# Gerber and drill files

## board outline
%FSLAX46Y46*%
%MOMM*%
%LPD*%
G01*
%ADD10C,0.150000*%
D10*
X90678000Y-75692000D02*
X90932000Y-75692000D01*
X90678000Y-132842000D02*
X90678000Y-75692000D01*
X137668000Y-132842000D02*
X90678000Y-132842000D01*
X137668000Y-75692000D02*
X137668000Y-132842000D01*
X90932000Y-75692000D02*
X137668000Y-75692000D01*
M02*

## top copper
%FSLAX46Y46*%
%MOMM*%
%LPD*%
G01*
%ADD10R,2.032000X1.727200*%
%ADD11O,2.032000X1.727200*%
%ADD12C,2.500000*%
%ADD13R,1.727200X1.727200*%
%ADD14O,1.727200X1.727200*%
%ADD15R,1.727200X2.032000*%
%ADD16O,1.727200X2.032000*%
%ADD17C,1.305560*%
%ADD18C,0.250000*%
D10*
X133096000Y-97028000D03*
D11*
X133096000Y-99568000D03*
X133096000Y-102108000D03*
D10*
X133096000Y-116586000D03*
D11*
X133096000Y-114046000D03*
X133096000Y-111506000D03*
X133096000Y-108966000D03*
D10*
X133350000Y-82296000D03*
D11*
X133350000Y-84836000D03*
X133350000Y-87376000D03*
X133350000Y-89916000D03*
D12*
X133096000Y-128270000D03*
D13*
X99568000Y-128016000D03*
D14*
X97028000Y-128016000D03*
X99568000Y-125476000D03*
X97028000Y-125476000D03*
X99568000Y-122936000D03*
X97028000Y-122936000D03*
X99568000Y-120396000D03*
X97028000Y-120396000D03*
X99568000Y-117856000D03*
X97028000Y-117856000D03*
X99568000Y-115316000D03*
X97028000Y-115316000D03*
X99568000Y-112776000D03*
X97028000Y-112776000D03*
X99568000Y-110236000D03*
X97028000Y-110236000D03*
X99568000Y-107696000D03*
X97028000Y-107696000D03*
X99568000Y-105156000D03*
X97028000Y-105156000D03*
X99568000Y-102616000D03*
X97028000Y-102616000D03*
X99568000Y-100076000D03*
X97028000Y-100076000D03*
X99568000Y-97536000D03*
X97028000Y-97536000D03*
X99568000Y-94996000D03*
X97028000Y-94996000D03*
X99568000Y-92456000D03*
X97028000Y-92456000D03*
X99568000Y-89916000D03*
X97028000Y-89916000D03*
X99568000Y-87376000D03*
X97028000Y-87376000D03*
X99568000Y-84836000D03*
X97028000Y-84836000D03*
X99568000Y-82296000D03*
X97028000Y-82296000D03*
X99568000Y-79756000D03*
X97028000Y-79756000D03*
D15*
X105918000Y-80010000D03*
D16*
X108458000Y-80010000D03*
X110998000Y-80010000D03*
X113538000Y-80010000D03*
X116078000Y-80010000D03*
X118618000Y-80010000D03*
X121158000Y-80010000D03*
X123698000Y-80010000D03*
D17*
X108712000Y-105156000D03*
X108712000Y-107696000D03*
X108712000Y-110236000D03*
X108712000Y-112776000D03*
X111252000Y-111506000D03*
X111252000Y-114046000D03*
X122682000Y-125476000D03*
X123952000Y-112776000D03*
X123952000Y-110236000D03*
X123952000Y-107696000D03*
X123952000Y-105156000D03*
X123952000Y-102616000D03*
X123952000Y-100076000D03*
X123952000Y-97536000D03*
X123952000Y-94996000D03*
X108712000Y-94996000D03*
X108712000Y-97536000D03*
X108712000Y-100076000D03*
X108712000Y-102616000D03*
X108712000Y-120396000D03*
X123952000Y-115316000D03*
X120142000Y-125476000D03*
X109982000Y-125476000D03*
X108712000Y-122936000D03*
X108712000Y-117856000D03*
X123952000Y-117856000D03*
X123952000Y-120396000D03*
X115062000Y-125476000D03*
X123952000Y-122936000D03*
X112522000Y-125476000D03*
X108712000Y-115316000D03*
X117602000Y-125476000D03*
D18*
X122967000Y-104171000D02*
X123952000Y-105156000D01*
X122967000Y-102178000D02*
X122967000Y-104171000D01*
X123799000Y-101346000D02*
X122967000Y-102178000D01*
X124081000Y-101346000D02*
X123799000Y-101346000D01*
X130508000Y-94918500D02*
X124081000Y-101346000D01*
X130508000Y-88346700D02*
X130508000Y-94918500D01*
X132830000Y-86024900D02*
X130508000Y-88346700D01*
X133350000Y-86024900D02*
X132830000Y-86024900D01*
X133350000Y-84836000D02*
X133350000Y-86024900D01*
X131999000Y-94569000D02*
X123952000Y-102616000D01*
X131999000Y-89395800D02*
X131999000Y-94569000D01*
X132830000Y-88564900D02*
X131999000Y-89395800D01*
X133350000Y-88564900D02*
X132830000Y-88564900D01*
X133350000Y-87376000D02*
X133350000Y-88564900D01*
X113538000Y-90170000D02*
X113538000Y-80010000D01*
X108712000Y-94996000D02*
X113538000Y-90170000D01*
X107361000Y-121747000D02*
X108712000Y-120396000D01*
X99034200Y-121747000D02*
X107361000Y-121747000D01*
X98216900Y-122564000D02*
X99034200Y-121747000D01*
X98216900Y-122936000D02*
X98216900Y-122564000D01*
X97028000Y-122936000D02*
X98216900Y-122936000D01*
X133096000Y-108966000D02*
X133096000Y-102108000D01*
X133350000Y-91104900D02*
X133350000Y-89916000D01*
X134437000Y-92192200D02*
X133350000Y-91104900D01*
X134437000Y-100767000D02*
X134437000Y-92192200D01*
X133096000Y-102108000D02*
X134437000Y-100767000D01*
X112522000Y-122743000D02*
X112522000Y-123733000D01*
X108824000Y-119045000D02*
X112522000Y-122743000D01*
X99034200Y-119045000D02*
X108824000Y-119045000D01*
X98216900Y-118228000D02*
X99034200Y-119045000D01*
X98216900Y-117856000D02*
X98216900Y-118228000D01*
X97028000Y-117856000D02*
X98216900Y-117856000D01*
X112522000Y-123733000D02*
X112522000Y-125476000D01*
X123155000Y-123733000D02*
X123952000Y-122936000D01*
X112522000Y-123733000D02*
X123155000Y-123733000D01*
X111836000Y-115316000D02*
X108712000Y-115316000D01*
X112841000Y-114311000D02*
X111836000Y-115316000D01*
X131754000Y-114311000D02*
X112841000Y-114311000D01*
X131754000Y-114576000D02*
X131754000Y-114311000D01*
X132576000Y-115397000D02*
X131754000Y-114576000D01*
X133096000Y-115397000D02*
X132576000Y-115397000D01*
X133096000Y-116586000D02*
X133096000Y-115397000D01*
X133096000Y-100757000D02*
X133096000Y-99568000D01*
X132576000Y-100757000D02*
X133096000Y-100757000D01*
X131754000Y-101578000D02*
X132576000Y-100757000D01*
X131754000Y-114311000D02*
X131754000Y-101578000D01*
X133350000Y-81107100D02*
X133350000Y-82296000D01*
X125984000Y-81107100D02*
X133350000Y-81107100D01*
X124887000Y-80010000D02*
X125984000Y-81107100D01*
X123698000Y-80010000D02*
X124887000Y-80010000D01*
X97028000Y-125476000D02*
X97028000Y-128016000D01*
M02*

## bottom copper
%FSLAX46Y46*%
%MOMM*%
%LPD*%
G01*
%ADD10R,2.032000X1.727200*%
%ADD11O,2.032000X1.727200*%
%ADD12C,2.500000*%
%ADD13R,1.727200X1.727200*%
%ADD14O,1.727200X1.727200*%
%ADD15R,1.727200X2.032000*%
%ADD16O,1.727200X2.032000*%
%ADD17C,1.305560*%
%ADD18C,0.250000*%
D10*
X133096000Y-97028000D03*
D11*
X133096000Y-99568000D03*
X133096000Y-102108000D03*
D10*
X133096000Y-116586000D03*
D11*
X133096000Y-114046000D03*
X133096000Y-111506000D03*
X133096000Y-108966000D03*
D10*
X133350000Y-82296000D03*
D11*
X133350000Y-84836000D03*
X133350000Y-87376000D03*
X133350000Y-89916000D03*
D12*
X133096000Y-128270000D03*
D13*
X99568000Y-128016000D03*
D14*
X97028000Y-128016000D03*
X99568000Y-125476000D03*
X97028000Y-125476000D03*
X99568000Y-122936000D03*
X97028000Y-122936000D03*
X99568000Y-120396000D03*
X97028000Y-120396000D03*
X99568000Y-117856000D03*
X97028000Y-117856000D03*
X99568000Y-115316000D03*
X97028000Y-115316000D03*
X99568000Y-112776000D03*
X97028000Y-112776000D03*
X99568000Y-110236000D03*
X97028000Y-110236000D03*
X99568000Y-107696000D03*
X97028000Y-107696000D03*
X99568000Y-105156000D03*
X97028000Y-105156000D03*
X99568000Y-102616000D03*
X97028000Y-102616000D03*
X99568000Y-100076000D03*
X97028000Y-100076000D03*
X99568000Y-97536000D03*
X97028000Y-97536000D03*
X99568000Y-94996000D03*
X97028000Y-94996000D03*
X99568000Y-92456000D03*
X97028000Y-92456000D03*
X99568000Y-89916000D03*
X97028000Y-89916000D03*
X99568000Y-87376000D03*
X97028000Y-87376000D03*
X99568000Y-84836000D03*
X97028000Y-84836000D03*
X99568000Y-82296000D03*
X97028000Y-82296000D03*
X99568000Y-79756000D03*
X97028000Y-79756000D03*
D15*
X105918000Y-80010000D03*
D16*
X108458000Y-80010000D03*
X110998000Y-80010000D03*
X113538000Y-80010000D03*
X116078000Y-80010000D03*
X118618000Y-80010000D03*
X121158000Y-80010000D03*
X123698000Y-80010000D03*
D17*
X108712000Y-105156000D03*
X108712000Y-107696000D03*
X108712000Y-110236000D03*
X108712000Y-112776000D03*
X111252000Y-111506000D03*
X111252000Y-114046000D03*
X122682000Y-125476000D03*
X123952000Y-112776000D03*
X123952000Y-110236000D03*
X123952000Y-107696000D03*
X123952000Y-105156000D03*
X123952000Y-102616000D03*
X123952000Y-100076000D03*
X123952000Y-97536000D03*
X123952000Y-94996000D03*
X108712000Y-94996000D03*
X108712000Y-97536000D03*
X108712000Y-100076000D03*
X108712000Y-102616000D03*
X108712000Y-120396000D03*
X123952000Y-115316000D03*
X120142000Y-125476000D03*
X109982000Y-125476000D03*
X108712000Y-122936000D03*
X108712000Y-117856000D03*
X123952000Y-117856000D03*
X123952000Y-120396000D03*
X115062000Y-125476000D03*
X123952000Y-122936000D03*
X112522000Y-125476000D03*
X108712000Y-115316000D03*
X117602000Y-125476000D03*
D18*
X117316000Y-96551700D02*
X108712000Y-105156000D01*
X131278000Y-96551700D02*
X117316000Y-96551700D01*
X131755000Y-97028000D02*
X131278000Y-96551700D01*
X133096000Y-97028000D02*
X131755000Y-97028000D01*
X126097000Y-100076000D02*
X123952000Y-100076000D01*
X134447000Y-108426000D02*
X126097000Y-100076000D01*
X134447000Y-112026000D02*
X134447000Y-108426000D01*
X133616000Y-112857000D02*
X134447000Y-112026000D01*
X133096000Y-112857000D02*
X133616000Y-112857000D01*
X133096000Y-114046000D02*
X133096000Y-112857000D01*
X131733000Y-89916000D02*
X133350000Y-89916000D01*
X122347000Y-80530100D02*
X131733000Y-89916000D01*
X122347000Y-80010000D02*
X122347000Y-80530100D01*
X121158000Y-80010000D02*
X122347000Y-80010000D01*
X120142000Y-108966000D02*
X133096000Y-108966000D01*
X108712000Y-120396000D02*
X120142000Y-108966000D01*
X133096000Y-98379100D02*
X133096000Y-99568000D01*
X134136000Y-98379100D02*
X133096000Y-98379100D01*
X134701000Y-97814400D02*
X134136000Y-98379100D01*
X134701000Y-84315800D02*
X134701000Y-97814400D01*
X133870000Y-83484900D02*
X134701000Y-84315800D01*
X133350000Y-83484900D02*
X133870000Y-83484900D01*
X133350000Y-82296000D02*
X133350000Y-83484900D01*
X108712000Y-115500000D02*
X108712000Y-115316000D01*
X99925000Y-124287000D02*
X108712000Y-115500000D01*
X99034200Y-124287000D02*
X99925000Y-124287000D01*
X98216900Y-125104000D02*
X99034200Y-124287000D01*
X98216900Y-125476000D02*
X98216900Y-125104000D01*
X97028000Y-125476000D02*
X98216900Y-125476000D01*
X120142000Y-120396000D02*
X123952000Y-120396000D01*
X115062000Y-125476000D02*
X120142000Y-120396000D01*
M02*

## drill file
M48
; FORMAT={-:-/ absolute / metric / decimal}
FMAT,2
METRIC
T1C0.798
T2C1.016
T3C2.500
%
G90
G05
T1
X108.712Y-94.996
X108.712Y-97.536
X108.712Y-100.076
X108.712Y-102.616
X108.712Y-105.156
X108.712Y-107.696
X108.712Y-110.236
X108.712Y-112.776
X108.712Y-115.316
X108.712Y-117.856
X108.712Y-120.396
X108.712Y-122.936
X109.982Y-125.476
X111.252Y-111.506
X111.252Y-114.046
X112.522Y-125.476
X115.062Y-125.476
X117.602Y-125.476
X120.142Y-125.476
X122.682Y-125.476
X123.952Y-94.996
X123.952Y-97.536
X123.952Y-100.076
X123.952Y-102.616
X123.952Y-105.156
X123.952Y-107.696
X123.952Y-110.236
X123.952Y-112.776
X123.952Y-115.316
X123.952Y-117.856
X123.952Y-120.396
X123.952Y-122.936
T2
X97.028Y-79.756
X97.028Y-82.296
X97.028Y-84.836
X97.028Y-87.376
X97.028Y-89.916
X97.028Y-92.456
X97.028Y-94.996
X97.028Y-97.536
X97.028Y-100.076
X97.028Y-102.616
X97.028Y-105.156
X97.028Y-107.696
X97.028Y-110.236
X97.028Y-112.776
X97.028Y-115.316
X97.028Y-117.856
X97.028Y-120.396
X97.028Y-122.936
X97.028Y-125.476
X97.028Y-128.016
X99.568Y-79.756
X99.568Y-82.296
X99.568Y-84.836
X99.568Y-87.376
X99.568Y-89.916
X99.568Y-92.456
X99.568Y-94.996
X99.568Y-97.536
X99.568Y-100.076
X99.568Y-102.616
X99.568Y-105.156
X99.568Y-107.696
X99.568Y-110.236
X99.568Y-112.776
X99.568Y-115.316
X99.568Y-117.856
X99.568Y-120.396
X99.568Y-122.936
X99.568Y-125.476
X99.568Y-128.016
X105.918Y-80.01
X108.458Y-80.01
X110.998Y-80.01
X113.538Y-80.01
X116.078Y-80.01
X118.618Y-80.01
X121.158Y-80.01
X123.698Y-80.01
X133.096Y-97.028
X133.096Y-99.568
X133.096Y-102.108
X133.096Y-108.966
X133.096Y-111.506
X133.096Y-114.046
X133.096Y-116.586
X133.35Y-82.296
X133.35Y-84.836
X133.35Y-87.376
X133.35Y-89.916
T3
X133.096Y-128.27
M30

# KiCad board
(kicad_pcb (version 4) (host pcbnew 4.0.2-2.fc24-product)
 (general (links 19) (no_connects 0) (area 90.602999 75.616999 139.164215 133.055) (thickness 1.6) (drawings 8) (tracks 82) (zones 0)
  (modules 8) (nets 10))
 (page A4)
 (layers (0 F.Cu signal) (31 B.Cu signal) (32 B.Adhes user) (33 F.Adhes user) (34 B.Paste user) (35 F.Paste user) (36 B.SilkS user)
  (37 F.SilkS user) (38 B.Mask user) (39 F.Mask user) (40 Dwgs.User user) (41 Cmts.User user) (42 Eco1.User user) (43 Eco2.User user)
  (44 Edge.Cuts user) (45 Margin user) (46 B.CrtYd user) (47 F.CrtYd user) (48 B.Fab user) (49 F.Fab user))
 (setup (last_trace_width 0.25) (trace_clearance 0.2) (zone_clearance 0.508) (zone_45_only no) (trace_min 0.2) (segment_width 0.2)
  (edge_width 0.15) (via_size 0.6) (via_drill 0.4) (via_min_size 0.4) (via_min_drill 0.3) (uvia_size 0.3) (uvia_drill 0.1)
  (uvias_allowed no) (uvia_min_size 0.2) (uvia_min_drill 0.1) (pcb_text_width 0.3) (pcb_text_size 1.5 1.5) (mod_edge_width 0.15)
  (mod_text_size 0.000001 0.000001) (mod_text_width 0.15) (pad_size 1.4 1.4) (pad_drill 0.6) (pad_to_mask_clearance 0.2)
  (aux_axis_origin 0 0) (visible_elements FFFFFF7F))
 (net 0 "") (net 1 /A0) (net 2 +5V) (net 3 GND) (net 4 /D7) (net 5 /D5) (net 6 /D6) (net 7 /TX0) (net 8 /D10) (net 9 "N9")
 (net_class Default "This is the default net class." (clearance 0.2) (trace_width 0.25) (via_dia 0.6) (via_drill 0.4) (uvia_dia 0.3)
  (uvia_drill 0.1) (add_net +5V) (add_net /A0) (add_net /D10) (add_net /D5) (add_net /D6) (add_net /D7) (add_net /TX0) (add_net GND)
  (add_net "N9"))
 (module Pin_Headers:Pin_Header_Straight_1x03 (layer F.Cu) (at 133.096 97.028)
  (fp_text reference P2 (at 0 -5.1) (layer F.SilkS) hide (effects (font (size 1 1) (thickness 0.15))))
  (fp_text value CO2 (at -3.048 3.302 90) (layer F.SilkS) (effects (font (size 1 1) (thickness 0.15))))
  (pad 1 thru_hole rect (at 0 0) (size 2.032 1.7272) (drill 1.016) (layers *.Cu *.Mask F.SilkS) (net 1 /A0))
  (pad 2 thru_hole oval (at 0 2.54) (size 2.032 1.7272) (drill 1.016) (layers *.Cu *.Mask F.SilkS) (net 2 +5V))
  (pad 3 thru_hole oval (at 0 5.08) (size 2.032 1.7272) (drill 1.016) (layers *.Cu *.Mask F.SilkS) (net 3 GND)))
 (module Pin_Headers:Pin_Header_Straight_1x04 (layer F.Cu) (at 133.096 116.586 180)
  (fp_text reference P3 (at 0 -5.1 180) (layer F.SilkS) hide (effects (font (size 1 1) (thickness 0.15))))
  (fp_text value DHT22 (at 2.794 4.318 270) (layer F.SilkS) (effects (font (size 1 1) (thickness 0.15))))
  (pad 1 thru_hole rect (at 0 0 180) (size 2.032 1.7272) (drill 1.016) (layers *.Cu *.Mask F.SilkS) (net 2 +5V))
  (pad 2 thru_hole oval (at 0 2.54 180) (size 2.032 1.7272) (drill 1.016) (layers *.Cu *.Mask F.SilkS) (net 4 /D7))
  (pad 3 thru_hole oval (at 0 5.08 180) (size 2.032 1.7272) (drill 1.016) (layers *.Cu *.Mask F.SilkS))
  (pad 4 thru_hole oval (at 0 7.62 180) (size 2.032 1.7272) (drill 1.016) (layers *.Cu *.Mask F.SilkS) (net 3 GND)))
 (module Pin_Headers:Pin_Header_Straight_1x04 (layer F.Cu) (at 133.35 82.296)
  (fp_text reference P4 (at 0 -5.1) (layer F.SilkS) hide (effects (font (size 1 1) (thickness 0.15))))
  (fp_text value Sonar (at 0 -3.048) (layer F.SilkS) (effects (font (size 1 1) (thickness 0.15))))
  (pad 1 thru_hole rect (at 0 0) (size 2.032 1.7272) (drill 1.016) (layers *.Cu *.Mask F.SilkS) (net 2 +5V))
  (pad 2 thru_hole oval (at 0 2.54) (size 2.032 1.7272) (drill 1.016) (layers *.Cu *.Mask F.SilkS) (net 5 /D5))
  (pad 3 thru_hole oval (at 0 5.08) (size 2.032 1.7272) (drill 1.016) (layers *.Cu *.Mask F.SilkS) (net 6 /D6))
  (pad 4 thru_hole oval (at 0 7.62) (size 2.032 1.7272) (drill 1.016) (layers *.Cu *.Mask F.SilkS) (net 3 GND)))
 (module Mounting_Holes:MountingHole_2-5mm (layer F.Cu) (at 133.096 128.27)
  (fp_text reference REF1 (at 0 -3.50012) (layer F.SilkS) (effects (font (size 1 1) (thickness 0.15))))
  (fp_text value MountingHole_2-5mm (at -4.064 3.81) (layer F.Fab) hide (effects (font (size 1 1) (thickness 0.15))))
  (pad 1 thru_hole circle (at 0 0) (size 2.5 2.5) (drill 2.5) (layers)))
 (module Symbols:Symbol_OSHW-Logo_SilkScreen (layer F.Cu) (at 126.746 84.582)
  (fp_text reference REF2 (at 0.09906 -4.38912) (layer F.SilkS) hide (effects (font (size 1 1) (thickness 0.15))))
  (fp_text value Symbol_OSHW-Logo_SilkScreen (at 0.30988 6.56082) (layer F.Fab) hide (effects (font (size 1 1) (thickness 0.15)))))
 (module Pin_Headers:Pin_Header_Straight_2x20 (layer F.Cu) (at 99.568 128.016 180)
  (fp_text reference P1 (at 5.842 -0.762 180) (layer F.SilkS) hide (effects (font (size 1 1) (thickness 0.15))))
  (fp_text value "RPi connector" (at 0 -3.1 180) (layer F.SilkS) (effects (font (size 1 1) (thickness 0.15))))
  (pad 1 thru_hole rect (at 0 0 180) (size 1.7272 1.7272) (drill 1.016) (layers *.Cu *.Mask F.SilkS))
  (pad 2 thru_hole oval (at 2.54 0 180) (size 1.7272 1.7272) (drill 1.016) (layers *.Cu *.Mask F.SilkS) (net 2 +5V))
  (pad 3 thru_hole oval (at 0 2.54 180) (size 1.7272 1.7272) (drill 1.016) (layers *.Cu *.Mask F.SilkS))
  (pad 4 thru_hole oval (at 2.54 2.54 180) (size 1.7272 1.7272) (drill 1.016) (layers *.Cu *.Mask F.SilkS) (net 2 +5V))
  (pad 5 thru_hole oval (at 0 5.08 180) (size 1.7272 1.7272) (drill 1.016) (layers *.Cu *.Mask F.SilkS))
  (pad 6 thru_hole oval (at 2.54 5.08 180) (size 1.7272 1.7272) (drill 1.016) (layers *.Cu *.Mask F.SilkS) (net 3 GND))
  (pad 7 thru_hole oval (at 0 7.62 180) (size 1.7272 1.7272) (drill 1.016) (layers *.Cu *.Mask F.SilkS))
  (pad 8 thru_hole oval (at 2.54 7.62 180) (size 1.7272 1.7272) (drill 1.016) (layers *.Cu *.Mask F.SilkS))
  (pad 9 thru_hole oval (at 0 10.16 180) (size 1.7272 1.7272) (drill 1.016) (layers *.Cu *.Mask F.SilkS))
  (pad 10 thru_hole oval (at 2.54 10.16 180) (size 1.7272 1.7272) (drill 1.016) (layers *.Cu *.Mask F.SilkS) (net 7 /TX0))
  (pad 11 thru_hole oval (at 0 12.7 180) (size 1.7272 1.7272) (drill 1.016) (layers *.Cu *.Mask F.SilkS))
  (pad 12 thru_hole oval (at 2.54 12.7 180) (size 1.7272 1.7272) (drill 1.016) (layers *.Cu *.Mask F.SilkS))
  (pad 13 thru_hole oval (at 0 15.24 180) (size 1.7272 1.7272) (drill 1.016) (layers *.Cu *.Mask F.SilkS))
  (pad 14 thru_hole oval (at 2.54 15.24 180) (size 1.7272 1.7272) (drill 1.016) (layers *.Cu *.Mask F.SilkS))
  (pad 15 thru_hole oval (at 0 17.78 180) (size 1.7272 1.7272) (drill 1.016) (layers *.Cu *.Mask F.SilkS))
  (pad 16 thru_hole oval (at 2.54 17.78 180) (size 1.7272 1.7272) (drill 1.016) (layers *.Cu *.Mask F.SilkS))
  (pad 17 thru_hole oval (at 0 20.32 180) (size 1.7272 1.7272) (drill 1.016) (layers *.Cu *.Mask F.SilkS))
  (pad 18 thru_hole oval (at 2.54 20.32 180) (size 1.7272 1.7272) (drill 1.016) (layers *.Cu *.Mask F.SilkS))
  (pad 19 thru_hole oval (at 0 22.86 180) (size 1.7272 1.7272) (drill 1.016) (layers *.Cu *.Mask F.SilkS))
  (pad 20 thru_hole oval (at 2.54 22.86 180) (size 1.7272 1.7272) (drill 1.016) (layers *.Cu *.Mask F.SilkS))
  (pad 21 thru_hole oval (at 0 25.4 180) (size 1.7272 1.7272) (drill 1.016) (layers *.Cu *.Mask F.SilkS))
  (pad 22 thru_hole oval (at 2.54 25.4 180) (size 1.7272 1.7272) (drill 1.016) (layers *.Cu *.Mask F.SilkS))
  (pad 23 thru_hole oval (at 0 27.94 180) (size 1.7272 1.7272) (drill 1.016) (layers *.Cu *.Mask F.SilkS))
  (pad 24 thru_hole oval (at 2.54 27.94 180) (size 1.7272 1.7272) (drill 1.016) (layers *.Cu *.Mask F.SilkS))
  (pad 25 thru_hole oval (at 0 30.48 180) (size 1.7272 1.7272) (drill 1.016) (layers *.Cu *.Mask F.SilkS))
  (pad 26 thru_hole oval (at 2.54 30.48 180) (size 1.7272 1.7272) (drill 1.016) (layers *.Cu *.Mask F.SilkS))
  (pad 27 thru_hole oval (at 0 33.02 180) (size 1.7272 1.7272) (drill 1.016) (layers *.Cu *.Mask F.SilkS))
  (pad 28 thru_hole oval (at 2.54 33.02 180) (size 1.7272 1.7272) (drill 1.016) (layers *.Cu *.Mask F.SilkS))
  (pad 29 thru_hole oval (at 0 35.56 180) (size 1.7272 1.7272) (drill 1.016) (layers *.Cu *.Mask F.SilkS))
  (pad 30 thru_hole oval (at 2.54 35.56 180) (size 1.7272 1.7272) (drill 1.016) (layers *.Cu *.Mask F.SilkS))
  (pad 31 thru_hole oval (at 0 38.1 180) (size 1.7272 1.7272) (drill 1.016) (layers *.Cu *.Mask F.SilkS))
  (pad 32 thru_hole oval (at 2.54 38.1 180) (size 1.7272 1.7272) (drill 1.016) (layers *.Cu *.Mask F.SilkS))
  (pad 33 thru_hole oval (at 0 40.64 180) (size 1.7272 1.7272) (drill 1.016) (layers *.Cu *.Mask F.SilkS))
  (pad 34 thru_hole oval (at 2.54 40.64 180) (size 1.7272 1.7272) (drill 1.016) (layers *.Cu *.Mask F.SilkS))
  (pad 35 thru_hole oval (at 0 43.18 180) (size 1.7272 1.7272) (drill 1.016) (layers *.Cu *.Mask F.SilkS))
  (pad 36 thru_hole oval (at 2.54 43.18 180) (size 1.7272 1.7272) (drill 1.016) (layers *.Cu *.Mask F.SilkS))
  (pad 37 thru_hole oval (at 0 45.72 180) (size 1.7272 1.7272) (drill 1.016) (layers *.Cu *.Mask F.SilkS))
  (pad 38 thru_hole oval (at 2.54 45.72 180) (size 1.7272 1.7272) (drill 1.016) (layers *.Cu *.Mask F.SilkS))
  (pad 39 thru_hole oval (at 0 48.26 180) (size 1.7272 1.7272) (drill 1.016) (layers *.Cu *.Mask F.SilkS))
  (pad 40 thru_hole oval (at 2.54 48.26 180) (size 1.7272 1.7272) (drill 1.016) (layers *.Cu *.Mask F.SilkS)))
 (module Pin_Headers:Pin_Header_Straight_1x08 (layer F.Cu) (at 105.918 80.01 90)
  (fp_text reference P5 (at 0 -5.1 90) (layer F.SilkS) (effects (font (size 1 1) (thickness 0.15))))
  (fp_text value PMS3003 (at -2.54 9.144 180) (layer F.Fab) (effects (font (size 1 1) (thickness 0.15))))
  (pad 1 thru_hole rect (at 0 0 90) (size 2.032 1.7272) (drill 1.016) (layers *.Cu *.Mask F.SilkS))
  (pad 2 thru_hole oval (at 0 2.54 90) (size 2.032 1.7272) (drill 1.016) (layers *.Cu *.Mask F.SilkS))
  (pad 3 thru_hole oval (at 0 5.08 90) (size 2.032 1.7272) (drill 1.016) (layers *.Cu *.Mask F.SilkS))
  (pad 4 thru_hole oval (at 0 7.62 90) (size 2.032 1.7272) (drill 1.016) (layers *.Cu *.Mask F.SilkS) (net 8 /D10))
  (pad 5 thru_hole oval (at 0 10.16 90) (size 2.032 1.7272) (drill 1.016) (layers *.Cu *.Mask F.SilkS))
  (pad 6 thru_hole oval (at 0 12.7 90) (size 2.032 1.7272) (drill 1.016) (layers *.Cu *.Mask F.SilkS))
  (pad 7 thru_hole oval (at 0 15.24 90) (size 2.032 1.7272) (drill 1.016) (layers *.Cu *.Mask F.SilkS) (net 3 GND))
  (pad 8 thru_hole oval (at 0 17.78 90) (size 2.032 1.7272) (drill 1.016) (layers *.Cu *.Mask F.SilkS) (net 2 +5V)))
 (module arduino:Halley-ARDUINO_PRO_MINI (layer F.Cu) (at 116.332 111.506 270)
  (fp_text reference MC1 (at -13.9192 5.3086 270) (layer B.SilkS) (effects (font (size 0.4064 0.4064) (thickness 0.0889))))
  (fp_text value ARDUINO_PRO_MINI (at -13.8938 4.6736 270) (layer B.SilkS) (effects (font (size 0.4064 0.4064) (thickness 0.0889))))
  (pad A0 thru_hole circle (at -6.35 7.62 270) (size 1.30556 1.30556) (drill 0.79756) (layers *.Cu F.Paste F.SilkS F.Mask) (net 1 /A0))
  (pad A1 thru_hole circle (at -3.81 7.62 270) (size 1.30556 1.30556) (drill 0.79756) (layers *.Cu F.Paste F.SilkS F.Mask))
  (pad A2 thru_hole circle (at -1.27 7.62 270) (size 1.30556 1.30556) (drill 0.79756) (layers *.Cu F.Paste F.SilkS F.Mask))
  (pad A3 thru_hole circle (at 1.27 7.62 270) (size 1.30556 1.30556) (drill 0.79756) (layers *.Cu F.Paste F.SilkS F.Mask))
  (pad A4 thru_hole circle (at 0 5.08 270) (size 1.30556 1.30556) (drill 0.79756) (layers *.Cu F.Paste F.SilkS F.Mask))
  (pad A5 thru_hole circle (at 2.54 5.08 270) (size 1.30556 1.30556) (drill 0.79756) (layers *.Cu F.Paste F.SilkS F.Mask))
  (pad BLK thru_hole circle (at 13.97 -6.35 270) (size 1.30556 1.30556) (drill 0.79756) (layers *.Cu F.Paste F.SilkS F.Mask))
  (pad D2 thru_hole circle (at 1.27 -7.62 270) (size 1.30556 1.30556) (drill 0.79756) (layers *.Cu F.Paste F.SilkS F.Mask))
  (pad D3 thru_hole circle (at -1.27 -7.62 270) (size 1.30556 1.30556) (drill 0.79756) (layers *.Cu F.Paste F.SilkS F.Mask))
  (pad D4 thru_hole circle (at -3.81 -7.62 270) (size 1.30556 1.30556) (drill 0.79756) (layers *.Cu F.Paste F.SilkS F.Mask))
  (pad D5 thru_hole circle (at -6.35 -7.62 270) (size 1.30556 1.30556) (drill 0.79756) (layers *.Cu F.Paste F.SilkS F.Mask) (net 5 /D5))
  (pad D6 thru_hole circle (at -8.89 -7.62 270) (size 1.30556 1.30556) (drill 0.79756) (layers *.Cu F.Paste F.SilkS F.Mask) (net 6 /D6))
  (pad D7 thru_hole circle (at -11.43 -7.62 270) (size 1.30556 1.30556) (drill 0.79756) (layers *.Cu F.Paste F.SilkS F.Mask) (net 4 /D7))
  (pad D8 thru_hole circle (at -13.97 -7.62 270) (size 1.30556 1.30556) (drill 0.79756) (layers *.Cu F.Paste F.SilkS F.Mask))
  (pad D9 thru_hole circle (at -16.51 -7.62 270) (size 1.30556 1.30556) (drill 0.79756) (layers *.Cu F.Paste F.SilkS F.Mask))
  (pad D10 thru_hole circle (at -16.51 7.62 270) (size 1.30556 1.30556) (drill 0.79756) (layers *.Cu F.Paste F.SilkS F.Mask) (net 8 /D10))
  (pad D11 thru_hole circle (at -13.97 7.62 270) (size 1.30556 1.30556) (drill 0.79756) (layers *.Cu F.Paste F.SilkS F.Mask))
  (pad D12 thru_hole circle (at -11.43 7.62 270) (size 1.30556 1.30556) (drill 0.79756) (layers *.Cu F.Paste F.SilkS F.Mask))
  (pad D13 thru_hole circle (at -8.89 7.62 270) (size 1.30556 1.30556) (drill 0.79756) (layers *.Cu F.Paste F.SilkS F.Mask))
  (pad GND1 thru_hole circle (at 8.89 7.62 270) (size 1.30556 1.30556) (drill 0.79756) (layers *.Cu F.Paste F.SilkS F.Mask) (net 3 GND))
  (pad GND2 thru_hole circle (at 3.81 -7.62 270) (size 1.30556 1.30556) (drill 0.79756) (layers *.Cu F.Paste F.SilkS F.Mask))
  (pad CTS thru_hole circle (at 13.97 -3.81 270) (size 1.30556 1.30556) (drill 0.79756) (layers *.Cu F.Paste F.SilkS F.Mask))
  (pad GRN thru_hole circle (at 13.97 6.35 270) (size 1.30556 1.30556) (drill 0.79756) (layers *.Cu F.Paste F.SilkS F.Mask))
  (pad RAW thru_hole circle (at 11.43 7.62 270) (size 1.30556 1.30556) (drill 0.79756) (layers *.Cu F.Paste F.SilkS F.Mask))
  (pad RST1 thru_hole circle (at 6.35 7.62 270) (size 1.30556 1.30556) (drill 0.79756) (layers *.Cu F.Paste F.SilkS F.Mask))
  (pad RST2 thru_hole circle (at 6.35 -7.62 270) (size 1.30556 1.30556) (drill 0.79756) (layers *.Cu F.Paste F.SilkS F.Mask))
  (pad RXI thru_hole circle (at 8.89 -7.62 270) (size 1.30556 1.30556) (drill 0.79756) (layers *.Cu F.Paste F.SilkS F.Mask) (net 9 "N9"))
  (pad RXI thru_hole circle (at 13.97 1.27 270) (size 1.30556 1.30556) (drill 0.79756) (layers *.Cu F.Paste F.SilkS F.Mask) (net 9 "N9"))
  (pad TXO thru_hole circle (at 11.43 -7.62 270) (size 1.30556 1.30556) (drill 0.79756) (layers *.Cu F.Paste F.SilkS F.Mask) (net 7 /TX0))
  (pad TXO thru_hole circle (at 13.97 3.81 270) (size 1.30556 1.30556) (drill 0.79756) (layers *.Cu F.Paste F.SilkS F.Mask) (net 7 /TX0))
  (pad VCC1 thru_hole circle (at 3.81 7.62 270) (size 1.30556 1.30556) (drill 0.79756) (layers *.Cu F.Paste F.SilkS F.Mask) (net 2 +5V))
  (pad VCC2 thru_hole circle (at 13.97 -1.27 270) (size 1.30556 1.30556) (drill 0.79756) (layers *.Cu F.Paste F.SilkS F.Mask)))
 (gr_line (start 90.678 75.692) (end 90.932 75.692) (angle 90) (layer Edge.Cuts) (width 0.15))
 (gr_line (start 90.678 132.842) (end 90.678 75.692) (angle 90) (layer Edge.Cuts) (width 0.15))
 (gr_line (start 137.668 132.842) (end 90.678 132.842) (angle 90) (layer Edge.Cuts) (width 0.15))
 (gr_line (start 137.668 75.692) (end 137.668 132.842) (angle 90) (layer Edge.Cuts) (width 0.15))
 (gr_line (start 90.932 75.692) (end 137.668 75.692) (angle 90) (layer Edge.Cuts) (width 0.15))
 (segment (start 117.316 96.5517) (end 108.712 105.156) (width 0.25) (layer B.Cu) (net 1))
 (segment (start 131.278 96.5517) (end 117.316 96.5517) (width 0.25) (layer B.Cu) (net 1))
 (segment (start 131.755 97.028) (end 131.278 96.5517) (width 0.25) (layer B.Cu) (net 1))
 (segment (start 133.096 97.028) (end 131.755 97.028) (width 0.25) (layer B.Cu) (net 1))
 (segment (start 122.967 104.171) (end 123.952 105.156) (width 0.25) (layer F.Cu) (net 5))
 (segment (start 122.967 102.178) (end 122.967 104.171) (width 0.25) (layer F.Cu) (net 5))
 (segment (start 123.799 101.346) (end 122.967 102.178) (width 0.25) (layer F.Cu) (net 5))
 (segment (start 124.081 101.346) (end 123.799 101.346) (width 0.25) (layer F.Cu) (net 5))
 (segment (start 130.508 94.9185) (end 124.081 101.346) (width 0.25) (layer F.Cu) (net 5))
 (segment (start 130.508 88.3467) (end 130.508 94.9185) (width 0.25) (layer F.Cu) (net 5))
 (segment (start 132.83 86.0249) (end 130.508 88.3467) (width 0.25) (layer F.Cu) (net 5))
 (segment (start 133.35 86.0249) (end 132.83 86.0249) (width 0.25) (layer F.Cu) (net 5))
 (segment (start 133.35 84.836) (end 133.35 86.0249) (width 0.25) (layer F.Cu) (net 5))
 (segment (start 131.999 94.569) (end 123.952 102.616) (width 0.25) (layer F.Cu) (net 6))
 (segment (start 131.999 89.3958) (end 131.999 94.569) (width 0.25) (layer F.Cu) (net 6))
 (segment (start 132.83 88.5649) (end 131.999 89.3958) (width 0.25) (layer F.Cu) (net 6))
 (segment (start 133.35 88.5649) (end 132.83 88.5649) (width 0.25) (layer F.Cu) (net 6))
 (segment (start 133.35 87.376) (end 133.35 88.5649) (width 0.25) (layer F.Cu) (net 6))
 (segment (start 126.097 100.076) (end 123.952 100.076) (width 0.25) (layer B.Cu) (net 4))
 (segment (start 134.447 108.426) (end 126.097 100.076) (width 0.25) (layer B.Cu) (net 4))
 (segment (start 134.447 112.026) (end 134.447 108.426) (width 0.25) (layer B.Cu) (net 4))
 (segment (start 133.616 112.857) (end 134.447 112.026) (width 0.25) (layer B.Cu) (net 4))
 (segment (start 133.096 112.857) (end 133.616 112.857) (width 0.25) (layer B.Cu) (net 4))
 (segment (start 133.096 114.046) (end 133.096 112.857) (width 0.25) (layer B.Cu) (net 4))
 (segment (start 113.538 90.17) (end 113.538 80.01) (width 0.25) (layer F.Cu) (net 8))
 (segment (start 108.712 94.996) (end 113.538 90.17) (width 0.25) (layer F.Cu) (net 8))
 (segment (start 107.361 121.747) (end 108.712 120.396) (width 0.25) (layer F.Cu) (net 3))
 (segment (start 99.0342 121.747) (end 107.361 121.747) (width 0.25) (layer F.Cu) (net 3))
 (segment (start 98.2169 122.564) (end 99.0342 121.747) (width 0.25) (layer F.Cu) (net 3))
 (segment (start 98.2169 122.936) (end 98.2169 122.564) (width 0.25) (layer F.Cu) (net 3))
 (segment (start 97.028 122.936) (end 98.2169 122.936) (width 0.25) (layer F.Cu) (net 3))
 (segment (start 131.733 89.916) (end 133.35 89.916) (width 0.25) (layer B.Cu) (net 3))
 (segment (start 122.347 80.5301) (end 131.733 89.916) (width 0.25) (layer B.Cu) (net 3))
 (segment (start 122.347 80.01) (end 122.347 80.5301) (width 0.25) (layer B.Cu) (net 3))
 (segment (start 121.158 80.01) (end 122.347 80.01) (width 0.25) (layer B.Cu) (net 3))
 (segment (start 133.096 108.966) (end 133.096 102.108) (width 0.25) (layer F.Cu) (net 3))
 (segment (start 133.35 91.1049) (end 133.35 89.916) (width 0.25) (layer F.Cu) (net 3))
 (segment (start 134.437 92.1922) (end 133.35 91.1049) (width 0.25) (layer F.Cu) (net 3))
 (segment (start 134.437 100.767) (end 134.437 92.1922) (width 0.25) (layer F.Cu) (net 3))
 (segment (start 133.096 102.108) (end 134.437 100.767) (width 0.25) (layer F.Cu) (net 3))
 (segment (start 120.142 108.966) (end 133.096 108.966) (width 0.25) (layer B.Cu) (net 3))
 (segment (start 108.712 120.396) (end 120.142 108.966) (width 0.25) (layer B.Cu) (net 3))
 (segment (start 112.522 122.743) (end 112.522 123.733) (width 0.25) (layer F.Cu) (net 7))
 (segment (start 108.824 119.045) (end 112.522 122.743) (width 0.25) (layer F.Cu) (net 7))
 (segment (start 99.0342 119.045) (end 108.824 119.045) (width 0.25) (layer F.Cu) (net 7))
 (segment (start 98.2169 118.228) (end 99.0342 119.045) (width 0.25) (layer F.Cu) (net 7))
 (segment (start 98.2169 117.856) (end 98.2169 118.228) (width 0.25) (layer F.Cu) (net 7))
 (segment (start 97.028 117.856) (end 98.2169 117.856) (width 0.25) (layer F.Cu) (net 7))
 (segment (start 112.522 123.733) (end 112.522 125.476) (width 0.25) (layer F.Cu) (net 7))
 (segment (start 123.155 123.733) (end 123.952 122.936) (width 0.25) (layer F.Cu) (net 7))
 (segment (start 112.522 123.733) (end 123.155 123.733) (width 0.25) (layer F.Cu) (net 7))
 (segment (start 133.096 98.3791) (end 133.096 99.568) (width 0.25) (layer B.Cu) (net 2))
 (segment (start 134.136 98.3791) (end 133.096 98.3791) (width 0.25) (layer B.Cu) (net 2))
 (segment (start 134.701 97.8144) (end 134.136 98.3791) (width 0.25) (layer B.Cu) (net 2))
 (segment (start 134.701 84.3158) (end 134.701 97.8144) (width 0.25) (layer B.Cu) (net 2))
 (segment (start 133.87 83.4849) (end 134.701 84.3158) (width 0.25) (layer B.Cu) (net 2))
 (segment (start 133.35 83.4849) (end 133.87 83.4849) (width 0.25) (layer B.Cu) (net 2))
 (segment (start 133.35 82.296) (end 133.35 83.4849) (width 0.25) (layer B.Cu) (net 2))
 (segment (start 108.712 115.5) (end 108.712 115.316) (width 0.25) (layer B.Cu) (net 2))
 (segment (start 99.925 124.287) (end 108.712 115.5) (width 0.25) (layer B.Cu) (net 2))
 (segment (start 99.0342 124.287) (end 99.925 124.287) (width 0.25) (layer B.Cu) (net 2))
 (segment (start 98.2169 125.104) (end 99.0342 124.287) (width 0.25) (layer B.Cu) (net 2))
 (segment (start 98.2169 125.476) (end 98.2169 125.104) (width 0.25) (layer B.Cu) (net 2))
 (segment (start 97.028 125.476) (end 98.2169 125.476) (width 0.25) (layer B.Cu) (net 2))
 (segment (start 111.836 115.316) (end 108.712 115.316) (width 0.25) (layer F.Cu) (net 2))
 (segment (start 112.841 114.311) (end 111.836 115.316) (width 0.25) (layer F.Cu) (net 2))
 (segment (start 131.754 114.311) (end 112.841 114.311) (width 0.25) (layer F.Cu) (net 2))
 (segment (start 131.754 114.576) (end 131.754 114.311) (width 0.25) (layer F.Cu) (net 2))
 (segment (start 132.576 115.397) (end 131.754 114.576) (width 0.25) (layer F.Cu) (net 2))
 (segment (start 133.096 115.397) (end 132.576 115.397) (width 0.25) (layer F.Cu) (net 2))
 (segment (start 133.096 116.586) (end 133.096 115.397) (width 0.25) (layer F.Cu) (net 2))
 (segment (start 133.096 100.757) (end 133.096 99.568) (width 0.25) (layer F.Cu) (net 2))
 (segment (start 132.576 100.757) (end 133.096 100.757) (width 0.25) (layer F.Cu) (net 2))
 (segment (start 131.754 101.578) (end 132.576 100.757) (width 0.25) (layer F.Cu) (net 2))
 (segment (start 131.754 114.311) (end 131.754 101.578) (width 0.25) (layer F.Cu) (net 2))
 (segment (start 133.35 81.1071) (end 133.35 82.296) (width 0.25) (layer F.Cu) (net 2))
 (segment (start 125.984 81.1071) (end 133.35 81.1071) (width 0.25) (layer F.Cu) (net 2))
 (segment (start 124.887 80.01) (end 125.984 81.1071) (width 0.25) (layer F.Cu) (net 2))
 (segment (start 123.698 80.01) (end 124.887 80.01) (width 0.25) (layer F.Cu) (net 2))
 (segment (start 97.028 125.476) (end 97.028 128.016) (width 0.25) (layer F.Cu) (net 2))
 (segment (start 120.142 120.396) (end 123.952 120.396) (width 0.25) (layer B.Cu) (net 9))
 (segment (start 115.062 125.476) (end 120.142 120.396) (width 0.25) (layer B.Cu) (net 9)))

